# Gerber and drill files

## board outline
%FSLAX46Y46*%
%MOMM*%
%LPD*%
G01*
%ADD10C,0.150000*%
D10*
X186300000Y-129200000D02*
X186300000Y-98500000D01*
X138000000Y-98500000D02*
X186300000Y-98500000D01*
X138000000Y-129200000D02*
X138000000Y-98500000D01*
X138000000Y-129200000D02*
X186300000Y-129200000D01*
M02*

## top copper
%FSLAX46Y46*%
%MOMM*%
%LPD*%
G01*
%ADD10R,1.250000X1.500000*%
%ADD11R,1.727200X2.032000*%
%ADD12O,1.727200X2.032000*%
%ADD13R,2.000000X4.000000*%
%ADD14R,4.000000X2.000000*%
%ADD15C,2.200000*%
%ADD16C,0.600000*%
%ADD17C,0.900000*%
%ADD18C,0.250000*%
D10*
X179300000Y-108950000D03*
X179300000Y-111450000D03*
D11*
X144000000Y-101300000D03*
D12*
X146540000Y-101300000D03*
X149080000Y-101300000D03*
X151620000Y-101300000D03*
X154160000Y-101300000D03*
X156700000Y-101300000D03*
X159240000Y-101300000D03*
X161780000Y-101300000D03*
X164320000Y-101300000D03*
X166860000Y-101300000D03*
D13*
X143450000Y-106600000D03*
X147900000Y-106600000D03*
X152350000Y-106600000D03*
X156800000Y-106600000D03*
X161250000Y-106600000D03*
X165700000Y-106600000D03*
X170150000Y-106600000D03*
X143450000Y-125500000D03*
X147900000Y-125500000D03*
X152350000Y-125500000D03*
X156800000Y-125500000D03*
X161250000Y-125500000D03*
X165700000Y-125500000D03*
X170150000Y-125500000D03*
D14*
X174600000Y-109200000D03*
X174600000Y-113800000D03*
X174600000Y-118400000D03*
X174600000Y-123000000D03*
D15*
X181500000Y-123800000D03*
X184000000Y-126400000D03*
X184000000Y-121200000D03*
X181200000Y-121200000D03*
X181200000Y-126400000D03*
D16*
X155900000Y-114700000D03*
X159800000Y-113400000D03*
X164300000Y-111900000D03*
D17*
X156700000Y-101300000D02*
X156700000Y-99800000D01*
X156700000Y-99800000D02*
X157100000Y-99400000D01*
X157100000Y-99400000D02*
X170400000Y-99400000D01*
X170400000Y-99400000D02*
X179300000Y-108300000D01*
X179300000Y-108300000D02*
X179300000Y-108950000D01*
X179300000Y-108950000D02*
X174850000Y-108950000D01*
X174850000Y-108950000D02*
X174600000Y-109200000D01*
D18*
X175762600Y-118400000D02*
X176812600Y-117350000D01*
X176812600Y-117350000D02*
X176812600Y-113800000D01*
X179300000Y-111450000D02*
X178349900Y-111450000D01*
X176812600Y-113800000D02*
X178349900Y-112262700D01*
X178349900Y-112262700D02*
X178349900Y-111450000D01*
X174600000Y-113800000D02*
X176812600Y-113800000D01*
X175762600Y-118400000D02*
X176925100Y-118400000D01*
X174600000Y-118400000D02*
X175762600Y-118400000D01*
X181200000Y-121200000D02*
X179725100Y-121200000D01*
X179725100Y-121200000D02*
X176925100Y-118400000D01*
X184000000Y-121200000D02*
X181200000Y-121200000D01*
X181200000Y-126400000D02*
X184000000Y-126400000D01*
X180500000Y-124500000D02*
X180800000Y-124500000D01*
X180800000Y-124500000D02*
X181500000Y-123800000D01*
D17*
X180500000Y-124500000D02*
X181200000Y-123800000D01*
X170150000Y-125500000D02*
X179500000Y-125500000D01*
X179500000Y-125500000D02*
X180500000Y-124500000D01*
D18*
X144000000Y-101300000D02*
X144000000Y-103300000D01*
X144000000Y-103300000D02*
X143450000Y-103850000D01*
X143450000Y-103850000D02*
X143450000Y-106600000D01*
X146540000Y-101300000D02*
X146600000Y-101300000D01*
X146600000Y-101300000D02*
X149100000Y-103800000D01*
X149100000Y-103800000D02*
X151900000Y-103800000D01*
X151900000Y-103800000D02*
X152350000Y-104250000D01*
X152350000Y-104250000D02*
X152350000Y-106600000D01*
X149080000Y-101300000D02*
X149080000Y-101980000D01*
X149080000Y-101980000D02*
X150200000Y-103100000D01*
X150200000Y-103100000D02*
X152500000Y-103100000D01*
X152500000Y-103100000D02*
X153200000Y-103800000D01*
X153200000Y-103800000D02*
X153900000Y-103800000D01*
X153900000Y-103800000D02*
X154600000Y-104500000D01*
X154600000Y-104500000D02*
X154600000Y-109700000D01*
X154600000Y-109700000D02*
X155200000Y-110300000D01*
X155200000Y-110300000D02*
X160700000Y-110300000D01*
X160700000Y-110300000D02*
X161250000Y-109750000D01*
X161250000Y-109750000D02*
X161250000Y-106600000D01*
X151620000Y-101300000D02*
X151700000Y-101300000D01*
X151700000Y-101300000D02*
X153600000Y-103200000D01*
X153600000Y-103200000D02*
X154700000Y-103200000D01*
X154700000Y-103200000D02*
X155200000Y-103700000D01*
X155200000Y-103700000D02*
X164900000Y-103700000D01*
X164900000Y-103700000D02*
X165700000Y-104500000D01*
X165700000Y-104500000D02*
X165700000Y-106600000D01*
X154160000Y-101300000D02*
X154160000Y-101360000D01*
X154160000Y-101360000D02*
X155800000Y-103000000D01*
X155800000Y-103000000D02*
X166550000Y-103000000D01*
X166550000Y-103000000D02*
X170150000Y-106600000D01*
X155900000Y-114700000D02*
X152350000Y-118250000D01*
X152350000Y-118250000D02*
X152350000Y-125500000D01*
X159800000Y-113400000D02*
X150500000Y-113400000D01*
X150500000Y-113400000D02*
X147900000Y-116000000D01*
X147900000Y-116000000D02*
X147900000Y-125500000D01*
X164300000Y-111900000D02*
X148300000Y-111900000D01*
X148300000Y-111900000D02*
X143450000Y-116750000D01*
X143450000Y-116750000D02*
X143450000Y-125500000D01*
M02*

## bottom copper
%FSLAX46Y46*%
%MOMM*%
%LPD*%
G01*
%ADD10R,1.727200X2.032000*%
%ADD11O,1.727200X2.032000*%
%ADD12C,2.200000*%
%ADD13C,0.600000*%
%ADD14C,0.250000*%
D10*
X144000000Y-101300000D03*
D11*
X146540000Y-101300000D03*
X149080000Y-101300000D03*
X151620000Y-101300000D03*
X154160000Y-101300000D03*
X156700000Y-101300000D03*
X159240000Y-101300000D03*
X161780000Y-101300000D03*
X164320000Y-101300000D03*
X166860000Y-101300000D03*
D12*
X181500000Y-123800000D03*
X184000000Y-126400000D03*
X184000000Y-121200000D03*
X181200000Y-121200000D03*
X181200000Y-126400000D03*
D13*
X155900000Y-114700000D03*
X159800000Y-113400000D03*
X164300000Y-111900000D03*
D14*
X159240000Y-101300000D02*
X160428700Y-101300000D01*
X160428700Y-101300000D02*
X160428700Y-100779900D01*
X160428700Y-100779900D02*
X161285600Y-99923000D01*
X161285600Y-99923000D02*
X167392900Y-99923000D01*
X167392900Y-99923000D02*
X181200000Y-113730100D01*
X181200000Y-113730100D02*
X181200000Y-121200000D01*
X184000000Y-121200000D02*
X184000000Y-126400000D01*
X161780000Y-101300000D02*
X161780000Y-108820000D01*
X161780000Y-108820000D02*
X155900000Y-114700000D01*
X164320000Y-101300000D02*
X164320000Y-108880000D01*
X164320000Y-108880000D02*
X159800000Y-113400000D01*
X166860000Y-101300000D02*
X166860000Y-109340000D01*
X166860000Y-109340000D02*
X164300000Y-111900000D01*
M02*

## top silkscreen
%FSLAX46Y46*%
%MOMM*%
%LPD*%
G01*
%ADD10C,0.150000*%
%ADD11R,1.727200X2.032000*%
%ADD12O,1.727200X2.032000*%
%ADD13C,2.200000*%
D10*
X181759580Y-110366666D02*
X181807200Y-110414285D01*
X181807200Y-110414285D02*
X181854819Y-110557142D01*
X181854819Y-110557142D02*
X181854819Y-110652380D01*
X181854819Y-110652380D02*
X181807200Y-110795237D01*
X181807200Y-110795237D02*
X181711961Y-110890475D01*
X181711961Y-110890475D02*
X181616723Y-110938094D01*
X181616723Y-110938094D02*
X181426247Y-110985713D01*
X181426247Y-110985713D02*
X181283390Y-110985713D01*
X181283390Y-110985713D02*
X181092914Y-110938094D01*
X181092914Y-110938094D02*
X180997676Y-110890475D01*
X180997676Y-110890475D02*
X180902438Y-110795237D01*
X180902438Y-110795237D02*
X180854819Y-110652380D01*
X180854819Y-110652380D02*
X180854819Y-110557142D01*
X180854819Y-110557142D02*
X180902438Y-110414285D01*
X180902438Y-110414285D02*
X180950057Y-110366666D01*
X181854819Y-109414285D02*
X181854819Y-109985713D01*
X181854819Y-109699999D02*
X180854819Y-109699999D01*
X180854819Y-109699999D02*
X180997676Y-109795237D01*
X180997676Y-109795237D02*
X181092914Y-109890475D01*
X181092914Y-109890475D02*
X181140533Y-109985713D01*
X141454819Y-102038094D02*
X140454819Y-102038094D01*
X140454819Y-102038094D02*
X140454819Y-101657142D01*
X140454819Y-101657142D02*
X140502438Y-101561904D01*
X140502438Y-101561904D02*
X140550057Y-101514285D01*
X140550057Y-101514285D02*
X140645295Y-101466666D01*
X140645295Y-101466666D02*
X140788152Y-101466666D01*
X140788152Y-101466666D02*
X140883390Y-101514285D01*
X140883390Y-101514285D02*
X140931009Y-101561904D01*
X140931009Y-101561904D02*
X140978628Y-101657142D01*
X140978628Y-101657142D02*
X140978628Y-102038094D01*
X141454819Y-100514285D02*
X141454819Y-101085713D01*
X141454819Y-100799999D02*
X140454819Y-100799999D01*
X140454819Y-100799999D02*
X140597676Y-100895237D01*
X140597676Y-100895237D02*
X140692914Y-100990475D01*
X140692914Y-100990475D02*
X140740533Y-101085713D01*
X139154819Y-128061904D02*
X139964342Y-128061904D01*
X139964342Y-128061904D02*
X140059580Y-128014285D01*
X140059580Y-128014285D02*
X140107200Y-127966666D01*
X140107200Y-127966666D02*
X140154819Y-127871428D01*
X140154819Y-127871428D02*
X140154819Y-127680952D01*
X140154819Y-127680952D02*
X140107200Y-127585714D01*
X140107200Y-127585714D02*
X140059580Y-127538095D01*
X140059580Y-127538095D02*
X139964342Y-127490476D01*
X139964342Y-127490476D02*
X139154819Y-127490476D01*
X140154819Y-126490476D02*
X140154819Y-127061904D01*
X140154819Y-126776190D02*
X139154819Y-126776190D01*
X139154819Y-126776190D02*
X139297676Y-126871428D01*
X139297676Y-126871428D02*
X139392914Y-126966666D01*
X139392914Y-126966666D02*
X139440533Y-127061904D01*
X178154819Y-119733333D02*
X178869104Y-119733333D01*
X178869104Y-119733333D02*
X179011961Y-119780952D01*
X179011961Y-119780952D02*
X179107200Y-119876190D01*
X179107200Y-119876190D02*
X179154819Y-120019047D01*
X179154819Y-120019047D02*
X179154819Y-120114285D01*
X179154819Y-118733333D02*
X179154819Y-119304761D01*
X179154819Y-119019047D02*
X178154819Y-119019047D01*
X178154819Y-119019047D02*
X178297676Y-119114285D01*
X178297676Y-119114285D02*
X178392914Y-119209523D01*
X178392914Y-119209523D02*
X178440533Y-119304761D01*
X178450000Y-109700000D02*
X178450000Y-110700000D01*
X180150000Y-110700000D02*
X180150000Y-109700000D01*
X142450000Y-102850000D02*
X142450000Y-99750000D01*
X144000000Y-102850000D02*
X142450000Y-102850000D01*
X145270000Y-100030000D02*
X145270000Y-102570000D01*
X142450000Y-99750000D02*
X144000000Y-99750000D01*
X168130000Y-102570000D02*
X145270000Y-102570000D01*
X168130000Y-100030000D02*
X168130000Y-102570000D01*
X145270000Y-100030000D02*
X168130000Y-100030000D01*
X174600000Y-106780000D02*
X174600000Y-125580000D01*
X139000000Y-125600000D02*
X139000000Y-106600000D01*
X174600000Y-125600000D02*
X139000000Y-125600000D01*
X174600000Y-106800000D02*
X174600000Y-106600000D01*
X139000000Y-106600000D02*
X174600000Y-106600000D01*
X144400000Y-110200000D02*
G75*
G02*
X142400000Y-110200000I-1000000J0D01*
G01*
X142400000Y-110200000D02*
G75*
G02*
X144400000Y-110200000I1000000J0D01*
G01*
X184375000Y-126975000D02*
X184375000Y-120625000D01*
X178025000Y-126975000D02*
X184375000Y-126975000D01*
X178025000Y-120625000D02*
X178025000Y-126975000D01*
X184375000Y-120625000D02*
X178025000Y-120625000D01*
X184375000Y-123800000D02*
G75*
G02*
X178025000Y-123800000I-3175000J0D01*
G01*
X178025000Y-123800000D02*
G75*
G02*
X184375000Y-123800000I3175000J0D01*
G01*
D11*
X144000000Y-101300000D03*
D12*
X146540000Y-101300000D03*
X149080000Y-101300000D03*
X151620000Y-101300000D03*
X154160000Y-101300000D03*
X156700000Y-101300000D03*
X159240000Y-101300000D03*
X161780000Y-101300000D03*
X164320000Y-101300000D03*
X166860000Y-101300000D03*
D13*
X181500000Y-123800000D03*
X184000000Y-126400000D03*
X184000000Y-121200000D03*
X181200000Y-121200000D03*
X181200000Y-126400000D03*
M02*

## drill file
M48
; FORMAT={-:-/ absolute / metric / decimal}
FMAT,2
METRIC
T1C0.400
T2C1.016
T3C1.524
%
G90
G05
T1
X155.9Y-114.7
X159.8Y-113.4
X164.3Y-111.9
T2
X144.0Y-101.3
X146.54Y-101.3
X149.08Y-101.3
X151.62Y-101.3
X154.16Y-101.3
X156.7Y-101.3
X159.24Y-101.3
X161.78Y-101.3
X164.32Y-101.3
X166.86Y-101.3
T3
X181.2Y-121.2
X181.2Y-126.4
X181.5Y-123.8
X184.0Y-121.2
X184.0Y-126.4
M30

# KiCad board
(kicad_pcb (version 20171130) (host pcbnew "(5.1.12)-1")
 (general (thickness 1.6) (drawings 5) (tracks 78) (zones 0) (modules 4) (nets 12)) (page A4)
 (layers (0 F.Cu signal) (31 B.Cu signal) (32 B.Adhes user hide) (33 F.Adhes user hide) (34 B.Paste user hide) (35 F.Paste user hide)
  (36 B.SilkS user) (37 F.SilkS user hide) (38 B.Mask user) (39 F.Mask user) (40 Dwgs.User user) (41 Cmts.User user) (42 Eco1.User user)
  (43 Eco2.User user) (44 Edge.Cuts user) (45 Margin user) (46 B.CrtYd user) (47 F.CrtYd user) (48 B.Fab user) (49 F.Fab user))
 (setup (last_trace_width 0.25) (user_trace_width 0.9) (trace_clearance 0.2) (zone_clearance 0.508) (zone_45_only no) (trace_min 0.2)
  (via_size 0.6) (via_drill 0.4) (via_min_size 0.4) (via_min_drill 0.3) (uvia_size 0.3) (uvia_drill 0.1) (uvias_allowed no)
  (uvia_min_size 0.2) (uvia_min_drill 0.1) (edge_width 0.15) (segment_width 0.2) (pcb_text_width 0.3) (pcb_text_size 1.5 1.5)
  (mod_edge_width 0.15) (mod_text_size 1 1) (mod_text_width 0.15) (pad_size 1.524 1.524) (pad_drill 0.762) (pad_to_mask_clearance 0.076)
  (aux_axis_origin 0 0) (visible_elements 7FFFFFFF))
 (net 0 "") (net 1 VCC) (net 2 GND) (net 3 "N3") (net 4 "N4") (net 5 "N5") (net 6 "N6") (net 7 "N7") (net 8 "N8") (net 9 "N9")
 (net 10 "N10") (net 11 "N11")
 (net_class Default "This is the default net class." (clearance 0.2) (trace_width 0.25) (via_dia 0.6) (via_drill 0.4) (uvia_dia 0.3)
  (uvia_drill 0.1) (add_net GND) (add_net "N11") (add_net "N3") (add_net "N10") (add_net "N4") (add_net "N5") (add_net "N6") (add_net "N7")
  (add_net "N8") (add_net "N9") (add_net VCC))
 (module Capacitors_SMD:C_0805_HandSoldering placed (layer F.Cu) (at 179.3 110.2 270)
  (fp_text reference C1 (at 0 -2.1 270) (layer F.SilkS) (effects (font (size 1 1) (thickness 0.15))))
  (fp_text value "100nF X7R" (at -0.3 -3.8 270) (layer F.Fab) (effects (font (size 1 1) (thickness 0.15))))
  (fp_line (start -0.5 0.85) (end 0.5 0.85) (layer F.SilkS) (width 0.15))
  (fp_line (start 0.5 -0.85) (end -0.5 -0.85) (layer F.SilkS) (width 0.15))
  (pad 1 smd rect (at -1.25 0 270) (size 1.5 1.25) (layers F.Cu F.Paste F.Mask) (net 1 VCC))
  (pad 2 smd rect (at 1.25 0 270) (size 1.5 1.25) (layers F.Cu F.Paste F.Mask) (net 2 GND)))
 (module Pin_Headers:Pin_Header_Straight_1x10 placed (layer F.Cu) (at 144 101.3 90)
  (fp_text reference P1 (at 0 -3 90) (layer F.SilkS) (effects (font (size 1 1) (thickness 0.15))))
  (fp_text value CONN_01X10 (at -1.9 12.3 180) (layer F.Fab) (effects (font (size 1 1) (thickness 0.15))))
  (fp_line (start -1.55 -1.55) (end 1.55 -1.55) (layer F.SilkS) (width 0.15))
  (fp_line (start -1.55 0) (end -1.55 -1.55) (layer F.SilkS) (width 0.15))
  (fp_line (start 1.27 1.27) (end -1.27 1.27) (layer F.SilkS) (width 0.15))
  (fp_line (start 1.55 -1.55) (end 1.55 0) (layer F.SilkS) (width 0.15))
  (fp_line (start -1.27 24.13) (end -1.27 1.27) (layer F.SilkS) (width 0.15))
  (fp_line (start 1.27 24.13) (end -1.27 24.13) (layer F.SilkS) (width 0.15))
  (fp_line (start 1.27 1.27) (end 1.27 24.13) (layer F.SilkS) (width 0.15))
  (pad 1 thru_hole rect (at 0 0 90) (size 2.032 1.7272) (drill 1.016) (layers *.Cu *.Mask F.SilkS) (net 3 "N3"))
  (pad 2 thru_hole oval (at 0 2.54 90) (size 2.032 1.7272) (drill 1.016) (layers *.Cu *.Mask F.SilkS) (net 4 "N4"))
  (pad 3 thru_hole oval (at 0 5.08 90) (size 2.032 1.7272) (drill 1.016) (layers *.Cu *.Mask F.SilkS) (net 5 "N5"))
  (pad 4 thru_hole oval (at 0 7.62 90) (size 2.032 1.7272) (drill 1.016) (layers *.Cu *.Mask F.SilkS) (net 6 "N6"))
  (pad 5 thru_hole oval (at 0 10.16 90) (size 2.032 1.7272) (drill 1.016) (layers *.Cu *.Mask F.SilkS) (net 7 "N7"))
  (pad 6 thru_hole oval (at 0 12.7 90) (size 2.032 1.7272) (drill 1.016) (layers *.Cu *.Mask F.SilkS) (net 1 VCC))
  (pad 7 thru_hole oval (at 0 15.24 90) (size 2.032 1.7272) (drill 1.016) (layers *.Cu *.Mask F.SilkS) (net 2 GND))
  (pad 8 thru_hole oval (at 0 17.78 90) (size 2.032 1.7272) (drill 1.016) (layers *.Cu *.Mask F.SilkS) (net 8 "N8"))
  (pad 9 thru_hole oval (at 0 20.32 90) (size 2.032 1.7272) (drill 1.016) (layers *.Cu *.Mask F.SilkS) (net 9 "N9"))
  (pad 10 thru_hole oval (at 0 22.86 90) (size 2.032 1.7272) (drill 1.016) (layers *.Cu *.Mask F.SilkS) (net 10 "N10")))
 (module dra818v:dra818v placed (layer F.Cu) (at 139 106.6)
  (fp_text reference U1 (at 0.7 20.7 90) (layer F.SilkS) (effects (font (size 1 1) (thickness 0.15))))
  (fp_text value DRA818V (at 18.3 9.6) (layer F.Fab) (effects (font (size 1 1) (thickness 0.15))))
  (fp_line (start 35.6 0.18) (end 35.6 18.98) (layer F.SilkS) (width 0.15))
  (fp_line (start 0 19) (end 0 0) (layer F.SilkS) (width 0.15))
  (fp_line (start 35.6 19) (end 0 19) (layer F.SilkS) (width 0.15))
  (fp_line (start 35.6 0.2) (end 35.6 0) (layer F.SilkS) (width 0.15))
  (fp_line (start 0 0) (end 35.6 0) (layer F.SilkS) (width 0.15))
  (fp_circle (center 4.4 3.6) (end 3.4 3.6) (layer F.SilkS) (width 0.15))
  (pad 1 smd rect (at 4.45 0) (size 2 4) (layers F.Cu F.Paste F.Mask) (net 3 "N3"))
  (pad 2 smd rect (at 8.9 0) (size 2 4) (layers F.Cu F.Paste F.Mask))
  (pad 3 smd rect (at 13.35 0) (size 2 4) (layers F.Cu F.Paste F.Mask) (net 4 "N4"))
  (pad 4 smd rect (at 17.8 0) (size 2 4) (layers F.Cu F.Paste F.Mask))
  (pad 5 smd rect (at 22.25 0) (size 2 4) (layers F.Cu F.Paste F.Mask) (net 5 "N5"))
  (pad 6 smd rect (at 26.7 0) (size 2 4) (layers F.Cu F.Paste F.Mask) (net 6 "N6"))
  (pad 7 smd rect (at 31.15 0) (size 2 4) (layers F.Cu F.Paste F.Mask) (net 7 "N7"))
  (pad 18 smd rect (at 4.45 18.9) (size 2 4) (layers F.Cu F.Paste F.Mask) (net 10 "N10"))
  (pad 17 smd rect (at 8.9 18.9) (size 2 4) (layers F.Cu F.Paste F.Mask) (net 9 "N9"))
  (pad 16 smd rect (at 13.35 18.9) (size 2 4) (layers F.Cu F.Paste F.Mask) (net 8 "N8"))
  (pad 15 smd rect (at 17.8 18.9) (size 2 4) (layers F.Cu F.Paste F.Mask))
  (pad 14 smd rect (at 22.25 18.9) (size 2 4) (layers F.Cu F.Paste F.Mask))
  (pad 13 smd rect (at 26.7 18.9) (size 2 4) (layers F.Cu F.Paste F.Mask))
  (pad 12 smd rect (at 31.15 18.9) (size 2 4) (layers F.Cu F.Paste F.Mask) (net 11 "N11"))
  (pad 8 smd rect (at 35.6 2.6) (size 4 2) (layers F.Cu F.Paste F.Mask) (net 1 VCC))
  (pad 9 smd rect (at 35.6 7.2) (size 4 2) (layers F.Cu F.Paste F.Mask) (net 2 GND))
  (pad 10 smd rect (at 35.6 11.8) (size 4 2) (layers F.Cu F.Paste F.Mask) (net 2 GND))
  (pad 11 smd rect (at 35.6 16.4) (size 4 2) (layers F.Cu F.Paste F.Mask)))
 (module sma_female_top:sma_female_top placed (layer F.Cu) (at 181.2 123.8 270)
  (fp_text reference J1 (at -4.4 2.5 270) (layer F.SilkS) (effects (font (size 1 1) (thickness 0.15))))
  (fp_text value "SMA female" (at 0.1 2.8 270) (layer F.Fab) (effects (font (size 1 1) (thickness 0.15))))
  (fp_line (start 3.175 -3.175) (end -3.175 -3.175) (layer F.SilkS) (width 0.15))
  (fp_line (start 3.175 3.175) (end 3.175 -3.175) (layer F.SilkS) (width 0.15))
  (fp_line (start -3.175 3.175) (end 3.175 3.175) (layer F.SilkS) (width 0.15))
  (fp_line (start -3.175 -3.175) (end -3.175 3.175) (layer F.SilkS) (width 0.15))
  (fp_circle (center 0 0) (end 0 -3.175) (layer F.SilkS) (width 0.15))
  (pad 1 thru_hole circle (at 0 -0.3 270) (size 2.2 2.2) (drill 1.524) (layers *.Cu *.Mask F.SilkS) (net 11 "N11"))
  (pad 4 thru_hole circle (at 2.6 -2.8 270) (size 2.2 2.2) (drill 1.524) (layers *.Cu *.Mask F.SilkS) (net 2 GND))
  (pad 3 thru_hole circle (at -2.6 -2.8 270) (size 2.2 2.2) (drill 1.524) (layers *.Cu *.Mask F.SilkS) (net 2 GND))
  (pad 2 thru_hole circle (at -2.6 0 270) (size 2.2 2.2) (drill 1.524) (layers *.Cu *.Mask F.SilkS) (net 2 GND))
  (pad 5 thru_hole circle (at 2.6 0 270) (size 2.2 2.2) (drill 1.524) (layers *.Cu *.Mask F.SilkS) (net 2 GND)))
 (gr_line (start 186.3 129.2) (end 186.3 98.5) (angle 90) (layer Edge.Cuts) (width 0.15))
 (gr_line (start 138 98.5) (end 186.3 98.5) (angle 90) (layer Edge.Cuts) (width 0.15))
 (gr_line (start 138 129.2) (end 138 98.5) (angle 90) (layer Edge.Cuts) (width 0.15))
 (gr_line (start 138 129.2) (end 186.3 129.2) (angle 90) (layer Edge.Cuts) (width 0.15))
 (segment (start 156.7 101.3) (end 156.7 99.8) (width 0.9) (layer F.Cu) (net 1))
 (segment (start 156.7 99.8) (end 157.1 99.4) (width 0.9) (layer F.Cu) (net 1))
 (segment (start 157.1 99.4) (end 170.4 99.4) (width 0.9) (layer F.Cu) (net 1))
 (segment (start 170.4 99.4) (end 179.3 108.3) (width 0.9) (layer F.Cu) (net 1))
 (segment (start 179.3 108.3) (end 179.3 108.95) (width 0.9) (layer F.Cu) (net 1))
 (segment (start 179.3 108.95) (end 174.85 108.95) (width 0.9) (layer F.Cu) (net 1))
 (segment (start 174.85 108.95) (end 174.6 109.2) (width 0.9) (layer F.Cu) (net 1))
 (segment (start 159.24 101.3) (end 160.4287 101.3) (width 0.25) (layer B.Cu) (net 2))
 (segment (start 160.4287 101.3) (end 160.4287 100.7799) (width 0.25) (layer B.Cu) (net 2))
 (segment (start 160.4287 100.7799) (end 161.2856 99.923) (width 0.25) (layer B.Cu) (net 2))
 (segment (start 161.2856 99.923) (end 167.3929 99.923) (width 0.25) (layer B.Cu) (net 2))
 (segment (start 167.3929 99.923) (end 181.2 113.7301) (width 0.25) (layer B.Cu) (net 2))
 (segment (start 181.2 113.7301) (end 181.2 121.2) (width 0.25) (layer B.Cu) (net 2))
 (segment (start 175.7626 118.4) (end 176.8126 117.35) (width 0.25) (layer F.Cu) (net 2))
 (segment (start 176.8126 117.35) (end 176.8126 113.8) (width 0.25) (layer F.Cu) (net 2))
 (segment (start 179.3 111.45) (end 178.3499 111.45) (width 0.25) (layer F.Cu) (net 2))
 (segment (start 176.8126 113.8) (end 178.3499 112.2627) (width 0.25) (layer F.Cu) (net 2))
 (segment (start 178.3499 112.2627) (end 178.3499 111.45) (width 0.25) (layer F.Cu) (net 2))
 (segment (start 174.6 113.8) (end 176.8126 113.8) (width 0.25) (layer F.Cu) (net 2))
 (segment (start 175.7626 118.4) (end 176.9251 118.4) (width 0.25) (layer F.Cu) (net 2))
 (segment (start 174.6 118.4) (end 175.7626 118.4) (width 0.25) (layer F.Cu) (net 2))
 (segment (start 181.2 121.2) (end 179.7251 121.2) (width 0.25) (layer F.Cu) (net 2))
 (segment (start 179.7251 121.2) (end 176.9251 118.4) (width 0.25) (layer F.Cu) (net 2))
 (segment (start 184 121.2) (end 181.2 121.2) (width 0.25) (layer F.Cu) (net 2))
 (segment (start 184 121.2) (end 184 126.4) (width 0.25) (layer B.Cu) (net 2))
 (segment (start 181.2 126.4) (end 184 126.4) (width 0.25) (layer F.Cu) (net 2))
 (segment (start 180.5 124.5) (end 180.8 124.5) (width 0.25) (layer F.Cu) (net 11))
 (segment (start 180.8 124.5) (end 181.5 123.8) (width 0.25) (layer F.Cu) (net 11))
 (segment (start 180.5 124.5) (end 181.2 123.8) (width 0.9) (layer F.Cu) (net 11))
 (segment (start 170.15 125.5) (end 179.5 125.5) (width 0.9) (layer F.Cu) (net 11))
 (segment (start 179.5 125.5) (end 180.5 124.5) (width 0.9) (layer F.Cu) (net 11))
 (segment (start 144 101.3) (end 144 103.3) (width 0.25) (layer F.Cu) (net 3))
 (segment (start 144 103.3) (end 143.45 103.85) (width 0.25) (layer F.Cu) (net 3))
 (segment (start 143.45 103.85) (end 143.45 106.6) (width 0.25) (layer F.Cu) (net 3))
 (segment (start 146.54 101.3) (end 146.6 101.3) (width 0.25) (layer F.Cu) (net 4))
 (segment (start 146.6 101.3) (end 149.1 103.8) (width 0.25) (layer F.Cu) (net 4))
 (segment (start 149.1 103.8) (end 151.9 103.8) (width 0.25) (layer F.Cu) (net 4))
 (segment (start 151.9 103.8) (end 152.35 104.25) (width 0.25) (layer F.Cu) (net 4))
 (segment (start 152.35 104.25) (end 152.35 106.6) (width 0.25) (layer F.Cu) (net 4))
 (segment (start 149.08 101.3) (end 149.08 101.98) (width 0.25) (layer F.Cu) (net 5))
 (segment (start 149.08 101.98) (end 150.2 103.1) (width 0.25) (layer F.Cu) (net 5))
 (segment (start 150.2 103.1) (end 152.5 103.1) (width 0.25) (layer F.Cu) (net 5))
 (segment (start 152.5 103.1) (end 153.2 103.8) (width 0.25) (layer F.Cu) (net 5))
 (segment (start 153.2 103.8) (end 153.9 103.8) (width 0.25) (layer F.Cu) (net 5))
 (segment (start 153.9 103.8) (end 154.6 104.5) (width 0.25) (layer F.Cu) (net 5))
 (segment (start 154.6 104.5) (end 154.6 109.7) (width 0.25) (layer F.Cu) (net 5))
 (segment (start 154.6 109.7) (end 155.2 110.3) (width 0.25) (layer F.Cu) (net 5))
 (segment (start 155.2 110.3) (end 160.7 110.3) (width 0.25) (layer F.Cu) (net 5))
 (segment (start 160.7 110.3) (end 161.25 109.75) (width 0.25) (layer F.Cu) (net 5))
 (segment (start 161.25 109.75) (end 161.25 106.6) (width 0.25) (layer F.Cu) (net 5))
 (segment (start 151.62 101.3) (end 151.7 101.3) (width 0.25) (layer F.Cu) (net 6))
 (segment (start 151.7 101.3) (end 153.6 103.2) (width 0.25) (layer F.Cu) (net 6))
 (segment (start 153.6 103.2) (end 154.7 103.2) (width 0.25) (layer F.Cu) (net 6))
 (segment (start 154.7 103.2) (end 155.2 103.7) (width 0.25) (layer F.Cu) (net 6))
 (segment (start 155.2 103.7) (end 164.9 103.7) (width 0.25) (layer F.Cu) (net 6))
 (segment (start 164.9 103.7) (end 165.7 104.5) (width 0.25) (layer F.Cu) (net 6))
 (segment (start 165.7 104.5) (end 165.7 106.6) (width 0.25) (layer F.Cu) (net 6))
 (segment (start 154.16 101.3) (end 154.16 101.36) (width 0.25) (layer F.Cu) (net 7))
 (segment (start 154.16 101.36) (end 155.8 103) (width 0.25) (layer F.Cu) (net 7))
 (segment (start 155.8 103) (end 166.55 103) (width 0.25) (layer F.Cu) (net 7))
 (segment (start 166.55 103) (end 170.15 106.6) (width 0.25) (layer F.Cu) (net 7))
 (segment (start 155.9 114.7) (end 152.35 118.25) (width 0.25) (layer F.Cu) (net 8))
 (segment (start 152.35 118.25) (end 152.35 125.5) (width 0.25) (layer F.Cu) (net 8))
 (segment (start 161.78 101.3) (end 161.78 108.82) (width 0.25) (layer B.Cu) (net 8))
 (segment (start 161.78 108.82) (end 155.9 114.7) (width 0.25) (layer B.Cu) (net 8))
 (via (at 155.9 114.7) (size 0.6) (layers F.Cu B.Cu) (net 8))
 (segment (start 159.8 113.4) (end 150.5 113.4) (width 0.25) (layer F.Cu) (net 9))
 (segment (start 150.5 113.4) (end 147.9 116) (width 0.25) (layer F.Cu) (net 9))
 (segment (start 147.9 116) (end 147.9 125.5) (width 0.25) (layer F.Cu) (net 9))
 (segment (start 164.32 101.3) (end 164.32 108.88) (width 0.25) (layer B.Cu) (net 9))
 (segment (start 164.32 108.88) (end 159.8 113.4) (width 0.25) (layer B.Cu) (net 9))
 (via (at 159.8 113.4) (size 0.6) (layers F.Cu B.Cu) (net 9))
 (segment (start 166.86 101.3) (end 166.86 109.34) (width 0.25) (layer B.Cu) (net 10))
 (segment (start 166.86 109.34) (end 164.3 111.9) (width 0.25) (layer B.Cu) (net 10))
 (segment (start 164.3 111.9) (end 148.3 111.9) (width 0.25) (layer F.Cu) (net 10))
 (segment (start 148.3 111.9) (end 143.45 116.75) (width 0.25) (layer F.Cu) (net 10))
 (segment (start 143.45 116.75) (end 143.45 125.5) (width 0.25) (layer F.Cu) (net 10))
 (via (at 164.3 111.9) (size 0.6) (layers F.Cu B.Cu) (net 10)))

